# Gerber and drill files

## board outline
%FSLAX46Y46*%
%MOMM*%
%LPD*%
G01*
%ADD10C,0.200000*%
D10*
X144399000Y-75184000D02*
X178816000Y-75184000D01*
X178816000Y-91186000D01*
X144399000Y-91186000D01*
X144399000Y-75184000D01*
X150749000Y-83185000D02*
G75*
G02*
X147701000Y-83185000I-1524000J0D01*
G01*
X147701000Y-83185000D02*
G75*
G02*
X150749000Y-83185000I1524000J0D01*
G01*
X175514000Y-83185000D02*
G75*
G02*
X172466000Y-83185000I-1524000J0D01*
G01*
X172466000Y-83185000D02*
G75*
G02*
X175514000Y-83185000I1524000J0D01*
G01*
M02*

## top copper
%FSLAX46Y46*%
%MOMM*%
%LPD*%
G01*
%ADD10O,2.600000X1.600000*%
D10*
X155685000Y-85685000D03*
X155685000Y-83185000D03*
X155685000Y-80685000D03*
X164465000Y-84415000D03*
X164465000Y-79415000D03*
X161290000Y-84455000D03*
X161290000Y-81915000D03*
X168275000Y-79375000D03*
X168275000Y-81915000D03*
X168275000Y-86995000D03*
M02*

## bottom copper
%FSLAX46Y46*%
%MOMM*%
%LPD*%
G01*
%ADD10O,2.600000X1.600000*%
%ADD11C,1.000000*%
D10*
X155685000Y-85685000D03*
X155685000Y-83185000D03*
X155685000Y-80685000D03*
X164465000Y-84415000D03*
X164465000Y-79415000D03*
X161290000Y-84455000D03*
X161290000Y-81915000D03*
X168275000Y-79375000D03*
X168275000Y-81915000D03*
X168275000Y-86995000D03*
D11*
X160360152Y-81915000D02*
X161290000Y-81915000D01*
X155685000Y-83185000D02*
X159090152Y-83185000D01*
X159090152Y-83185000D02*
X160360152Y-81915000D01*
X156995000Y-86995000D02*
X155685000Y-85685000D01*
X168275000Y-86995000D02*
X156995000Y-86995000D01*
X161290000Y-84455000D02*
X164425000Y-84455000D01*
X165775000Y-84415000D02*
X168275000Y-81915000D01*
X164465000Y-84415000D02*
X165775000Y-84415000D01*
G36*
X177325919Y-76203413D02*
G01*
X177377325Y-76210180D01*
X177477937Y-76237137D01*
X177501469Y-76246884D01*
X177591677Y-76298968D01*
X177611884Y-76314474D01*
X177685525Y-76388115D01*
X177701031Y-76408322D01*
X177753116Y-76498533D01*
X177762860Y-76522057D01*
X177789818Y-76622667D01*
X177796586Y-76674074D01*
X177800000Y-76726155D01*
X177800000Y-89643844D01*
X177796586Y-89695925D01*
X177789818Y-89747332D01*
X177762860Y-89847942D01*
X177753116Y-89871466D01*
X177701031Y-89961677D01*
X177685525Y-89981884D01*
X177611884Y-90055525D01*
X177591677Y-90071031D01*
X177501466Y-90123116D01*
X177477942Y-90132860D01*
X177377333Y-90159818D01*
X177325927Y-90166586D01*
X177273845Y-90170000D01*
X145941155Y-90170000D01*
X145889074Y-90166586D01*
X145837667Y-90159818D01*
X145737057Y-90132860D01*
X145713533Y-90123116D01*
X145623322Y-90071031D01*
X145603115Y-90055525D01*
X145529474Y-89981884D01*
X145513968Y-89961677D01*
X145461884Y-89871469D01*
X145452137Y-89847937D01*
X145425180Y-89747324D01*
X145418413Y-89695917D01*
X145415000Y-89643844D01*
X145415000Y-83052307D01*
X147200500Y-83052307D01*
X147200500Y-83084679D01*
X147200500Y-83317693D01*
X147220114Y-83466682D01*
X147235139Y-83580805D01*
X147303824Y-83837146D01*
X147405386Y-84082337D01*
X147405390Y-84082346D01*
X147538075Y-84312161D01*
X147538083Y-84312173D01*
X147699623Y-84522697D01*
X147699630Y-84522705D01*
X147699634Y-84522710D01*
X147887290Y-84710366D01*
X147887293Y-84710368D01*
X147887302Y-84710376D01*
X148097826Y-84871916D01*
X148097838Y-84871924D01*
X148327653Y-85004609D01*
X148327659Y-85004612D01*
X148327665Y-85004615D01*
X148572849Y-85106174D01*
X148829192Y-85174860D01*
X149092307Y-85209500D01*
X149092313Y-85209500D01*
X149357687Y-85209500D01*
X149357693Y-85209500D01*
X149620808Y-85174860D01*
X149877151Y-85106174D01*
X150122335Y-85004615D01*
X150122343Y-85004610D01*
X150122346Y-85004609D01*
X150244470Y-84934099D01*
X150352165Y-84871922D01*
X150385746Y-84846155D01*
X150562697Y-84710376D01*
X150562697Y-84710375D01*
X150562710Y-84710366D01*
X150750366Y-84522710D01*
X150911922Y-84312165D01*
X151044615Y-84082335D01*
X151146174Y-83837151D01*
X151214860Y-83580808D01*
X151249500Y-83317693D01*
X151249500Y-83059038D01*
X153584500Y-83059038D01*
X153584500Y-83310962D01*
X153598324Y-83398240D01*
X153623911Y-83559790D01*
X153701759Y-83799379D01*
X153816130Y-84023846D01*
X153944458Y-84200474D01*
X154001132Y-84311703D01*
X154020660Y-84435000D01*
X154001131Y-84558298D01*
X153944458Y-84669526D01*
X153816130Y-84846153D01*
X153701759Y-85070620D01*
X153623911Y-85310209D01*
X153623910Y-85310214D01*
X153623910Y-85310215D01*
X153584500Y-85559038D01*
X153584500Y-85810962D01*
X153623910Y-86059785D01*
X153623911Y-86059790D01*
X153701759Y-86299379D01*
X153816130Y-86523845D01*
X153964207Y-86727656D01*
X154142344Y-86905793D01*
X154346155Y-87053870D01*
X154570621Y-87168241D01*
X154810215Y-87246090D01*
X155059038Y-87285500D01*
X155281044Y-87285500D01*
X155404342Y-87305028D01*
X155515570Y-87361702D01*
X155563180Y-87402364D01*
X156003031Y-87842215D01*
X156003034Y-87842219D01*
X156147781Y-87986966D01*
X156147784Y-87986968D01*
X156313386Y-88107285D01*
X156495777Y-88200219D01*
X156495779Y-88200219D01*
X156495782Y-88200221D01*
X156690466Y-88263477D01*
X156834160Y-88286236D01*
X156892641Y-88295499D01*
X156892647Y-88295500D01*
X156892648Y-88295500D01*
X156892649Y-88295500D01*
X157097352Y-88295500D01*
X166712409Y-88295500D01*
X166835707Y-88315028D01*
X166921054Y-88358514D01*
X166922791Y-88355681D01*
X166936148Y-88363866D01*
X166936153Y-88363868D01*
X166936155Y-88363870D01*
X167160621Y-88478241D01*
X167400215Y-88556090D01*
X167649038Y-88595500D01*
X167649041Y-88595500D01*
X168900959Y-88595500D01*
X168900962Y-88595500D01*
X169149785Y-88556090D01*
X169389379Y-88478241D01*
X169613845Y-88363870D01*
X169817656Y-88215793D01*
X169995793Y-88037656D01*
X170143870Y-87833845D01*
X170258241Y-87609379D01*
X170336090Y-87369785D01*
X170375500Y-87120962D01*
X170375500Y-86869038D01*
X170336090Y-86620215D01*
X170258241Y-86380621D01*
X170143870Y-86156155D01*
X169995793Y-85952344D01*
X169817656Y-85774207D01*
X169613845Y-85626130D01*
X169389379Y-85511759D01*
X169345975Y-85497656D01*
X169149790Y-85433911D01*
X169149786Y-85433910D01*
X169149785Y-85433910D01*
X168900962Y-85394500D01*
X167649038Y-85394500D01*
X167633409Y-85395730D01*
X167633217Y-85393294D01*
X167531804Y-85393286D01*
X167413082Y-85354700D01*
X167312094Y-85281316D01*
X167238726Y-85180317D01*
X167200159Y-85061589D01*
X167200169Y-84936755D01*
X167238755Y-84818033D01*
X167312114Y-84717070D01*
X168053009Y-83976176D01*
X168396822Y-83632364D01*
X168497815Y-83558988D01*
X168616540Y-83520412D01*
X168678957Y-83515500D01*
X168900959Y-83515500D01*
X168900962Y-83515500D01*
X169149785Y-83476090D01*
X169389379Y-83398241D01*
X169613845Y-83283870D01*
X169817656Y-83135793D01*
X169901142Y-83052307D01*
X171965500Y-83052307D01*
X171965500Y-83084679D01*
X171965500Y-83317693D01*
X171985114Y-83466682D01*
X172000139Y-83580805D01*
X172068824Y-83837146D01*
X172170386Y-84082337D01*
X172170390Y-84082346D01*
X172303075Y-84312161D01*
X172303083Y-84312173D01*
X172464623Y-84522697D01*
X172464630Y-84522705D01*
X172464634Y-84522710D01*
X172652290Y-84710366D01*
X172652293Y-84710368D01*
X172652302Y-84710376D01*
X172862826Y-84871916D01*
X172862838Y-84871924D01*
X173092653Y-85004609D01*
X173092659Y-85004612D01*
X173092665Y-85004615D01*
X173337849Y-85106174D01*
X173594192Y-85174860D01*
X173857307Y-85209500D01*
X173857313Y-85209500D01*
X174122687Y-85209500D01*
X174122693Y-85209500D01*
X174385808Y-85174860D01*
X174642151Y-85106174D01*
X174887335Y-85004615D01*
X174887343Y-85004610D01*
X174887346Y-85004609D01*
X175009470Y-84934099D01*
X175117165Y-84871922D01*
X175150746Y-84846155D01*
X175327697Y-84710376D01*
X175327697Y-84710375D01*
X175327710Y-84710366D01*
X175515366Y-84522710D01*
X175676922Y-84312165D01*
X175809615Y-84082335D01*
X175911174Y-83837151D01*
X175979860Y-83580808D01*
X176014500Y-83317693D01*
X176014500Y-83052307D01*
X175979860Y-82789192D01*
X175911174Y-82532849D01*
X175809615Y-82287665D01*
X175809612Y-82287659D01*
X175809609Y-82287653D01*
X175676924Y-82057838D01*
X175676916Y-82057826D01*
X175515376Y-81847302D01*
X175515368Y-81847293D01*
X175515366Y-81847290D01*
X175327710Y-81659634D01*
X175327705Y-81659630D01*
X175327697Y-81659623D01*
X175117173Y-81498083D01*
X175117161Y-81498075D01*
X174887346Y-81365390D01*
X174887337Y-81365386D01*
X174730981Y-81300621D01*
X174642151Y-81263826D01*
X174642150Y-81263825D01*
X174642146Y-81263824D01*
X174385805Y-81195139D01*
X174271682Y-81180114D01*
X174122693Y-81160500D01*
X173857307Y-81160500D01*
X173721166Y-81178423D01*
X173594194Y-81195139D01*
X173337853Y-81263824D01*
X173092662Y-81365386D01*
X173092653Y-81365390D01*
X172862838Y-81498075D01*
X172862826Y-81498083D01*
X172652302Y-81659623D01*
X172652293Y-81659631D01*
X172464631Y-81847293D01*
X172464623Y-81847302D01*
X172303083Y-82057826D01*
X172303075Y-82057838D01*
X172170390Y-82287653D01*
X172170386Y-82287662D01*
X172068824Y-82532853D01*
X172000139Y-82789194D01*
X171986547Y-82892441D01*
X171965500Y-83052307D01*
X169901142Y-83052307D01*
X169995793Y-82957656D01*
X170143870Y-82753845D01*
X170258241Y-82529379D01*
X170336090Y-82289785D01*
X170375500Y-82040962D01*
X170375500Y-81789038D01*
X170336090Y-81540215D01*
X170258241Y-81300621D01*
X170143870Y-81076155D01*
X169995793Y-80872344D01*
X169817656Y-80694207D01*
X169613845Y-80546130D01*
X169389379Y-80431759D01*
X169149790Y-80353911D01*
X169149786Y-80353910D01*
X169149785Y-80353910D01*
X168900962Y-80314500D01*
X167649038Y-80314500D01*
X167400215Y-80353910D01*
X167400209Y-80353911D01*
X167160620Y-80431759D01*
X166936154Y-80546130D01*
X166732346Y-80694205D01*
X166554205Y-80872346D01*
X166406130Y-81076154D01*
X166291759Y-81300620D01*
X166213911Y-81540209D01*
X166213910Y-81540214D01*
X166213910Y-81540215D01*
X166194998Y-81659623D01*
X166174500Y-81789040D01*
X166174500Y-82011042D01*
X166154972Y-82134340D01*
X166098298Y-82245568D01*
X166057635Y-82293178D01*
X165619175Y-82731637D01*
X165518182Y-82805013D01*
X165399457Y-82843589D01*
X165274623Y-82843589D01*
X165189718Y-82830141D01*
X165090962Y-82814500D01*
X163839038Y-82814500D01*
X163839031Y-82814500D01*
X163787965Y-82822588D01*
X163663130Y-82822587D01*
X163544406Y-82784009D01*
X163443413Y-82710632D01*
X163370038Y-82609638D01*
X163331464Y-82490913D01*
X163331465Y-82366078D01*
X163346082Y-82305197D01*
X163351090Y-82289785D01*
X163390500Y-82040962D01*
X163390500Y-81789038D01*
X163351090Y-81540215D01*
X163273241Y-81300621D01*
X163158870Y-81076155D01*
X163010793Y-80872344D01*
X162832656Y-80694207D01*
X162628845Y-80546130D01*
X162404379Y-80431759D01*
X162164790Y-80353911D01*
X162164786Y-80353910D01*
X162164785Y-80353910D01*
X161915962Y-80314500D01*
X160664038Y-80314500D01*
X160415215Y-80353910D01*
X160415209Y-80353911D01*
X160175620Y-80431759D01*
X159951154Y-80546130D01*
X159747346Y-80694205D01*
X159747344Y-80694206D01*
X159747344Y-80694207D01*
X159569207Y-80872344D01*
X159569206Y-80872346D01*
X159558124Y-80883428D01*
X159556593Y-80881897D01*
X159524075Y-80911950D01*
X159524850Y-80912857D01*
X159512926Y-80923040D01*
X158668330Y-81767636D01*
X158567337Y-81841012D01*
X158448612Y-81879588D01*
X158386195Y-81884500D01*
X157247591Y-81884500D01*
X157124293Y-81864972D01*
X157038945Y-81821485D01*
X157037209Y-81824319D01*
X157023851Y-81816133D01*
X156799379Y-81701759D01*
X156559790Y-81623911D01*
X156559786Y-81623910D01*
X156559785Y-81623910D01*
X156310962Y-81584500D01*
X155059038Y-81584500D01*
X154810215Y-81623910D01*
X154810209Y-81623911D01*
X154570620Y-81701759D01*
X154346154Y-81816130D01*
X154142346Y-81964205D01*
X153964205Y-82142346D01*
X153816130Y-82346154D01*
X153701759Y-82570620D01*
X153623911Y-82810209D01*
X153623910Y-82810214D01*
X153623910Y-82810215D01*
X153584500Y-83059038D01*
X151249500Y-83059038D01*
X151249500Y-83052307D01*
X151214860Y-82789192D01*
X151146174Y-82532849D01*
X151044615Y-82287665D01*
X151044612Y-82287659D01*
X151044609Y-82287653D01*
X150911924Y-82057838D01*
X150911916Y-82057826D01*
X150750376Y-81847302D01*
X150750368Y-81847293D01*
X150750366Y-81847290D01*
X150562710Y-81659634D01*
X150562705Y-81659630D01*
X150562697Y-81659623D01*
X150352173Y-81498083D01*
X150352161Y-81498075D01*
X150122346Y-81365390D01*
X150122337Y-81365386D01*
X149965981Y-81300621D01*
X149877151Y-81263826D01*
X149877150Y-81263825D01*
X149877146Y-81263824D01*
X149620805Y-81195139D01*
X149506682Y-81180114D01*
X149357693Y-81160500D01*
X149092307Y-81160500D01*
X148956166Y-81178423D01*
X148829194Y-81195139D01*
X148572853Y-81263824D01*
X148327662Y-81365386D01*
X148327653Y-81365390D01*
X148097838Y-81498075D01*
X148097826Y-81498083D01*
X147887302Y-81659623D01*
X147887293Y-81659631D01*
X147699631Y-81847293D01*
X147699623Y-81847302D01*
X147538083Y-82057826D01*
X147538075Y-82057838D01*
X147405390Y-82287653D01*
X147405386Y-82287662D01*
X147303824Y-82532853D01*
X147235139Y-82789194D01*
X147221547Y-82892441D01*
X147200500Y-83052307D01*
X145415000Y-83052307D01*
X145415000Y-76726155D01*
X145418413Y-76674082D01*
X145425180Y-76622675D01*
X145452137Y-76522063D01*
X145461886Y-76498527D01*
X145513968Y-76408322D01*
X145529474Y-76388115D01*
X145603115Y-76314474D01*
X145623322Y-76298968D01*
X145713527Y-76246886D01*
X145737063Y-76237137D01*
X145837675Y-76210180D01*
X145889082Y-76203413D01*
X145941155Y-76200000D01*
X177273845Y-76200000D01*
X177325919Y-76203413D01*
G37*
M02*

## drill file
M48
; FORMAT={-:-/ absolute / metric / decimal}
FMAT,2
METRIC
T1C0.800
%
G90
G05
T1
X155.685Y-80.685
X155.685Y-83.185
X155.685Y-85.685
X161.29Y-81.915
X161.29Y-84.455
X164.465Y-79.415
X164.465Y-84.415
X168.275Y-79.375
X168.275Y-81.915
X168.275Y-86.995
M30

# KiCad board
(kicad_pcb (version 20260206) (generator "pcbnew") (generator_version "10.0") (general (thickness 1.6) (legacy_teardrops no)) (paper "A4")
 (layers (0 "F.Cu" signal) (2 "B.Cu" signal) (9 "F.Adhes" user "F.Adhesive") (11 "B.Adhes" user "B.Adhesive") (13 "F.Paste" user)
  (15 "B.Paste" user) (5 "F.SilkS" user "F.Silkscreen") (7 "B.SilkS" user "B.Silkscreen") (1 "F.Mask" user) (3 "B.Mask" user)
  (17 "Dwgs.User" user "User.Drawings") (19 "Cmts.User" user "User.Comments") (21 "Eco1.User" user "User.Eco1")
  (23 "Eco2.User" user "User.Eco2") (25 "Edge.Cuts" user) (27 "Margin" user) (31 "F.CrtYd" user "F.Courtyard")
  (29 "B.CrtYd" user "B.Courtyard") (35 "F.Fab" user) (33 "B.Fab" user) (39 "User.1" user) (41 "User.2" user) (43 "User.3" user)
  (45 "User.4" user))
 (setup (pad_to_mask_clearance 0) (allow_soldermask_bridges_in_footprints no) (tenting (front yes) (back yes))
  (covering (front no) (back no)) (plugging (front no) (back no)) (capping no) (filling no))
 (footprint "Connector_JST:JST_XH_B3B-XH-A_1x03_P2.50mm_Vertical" (layer "F.Cu") (at 155.685 85.685 90)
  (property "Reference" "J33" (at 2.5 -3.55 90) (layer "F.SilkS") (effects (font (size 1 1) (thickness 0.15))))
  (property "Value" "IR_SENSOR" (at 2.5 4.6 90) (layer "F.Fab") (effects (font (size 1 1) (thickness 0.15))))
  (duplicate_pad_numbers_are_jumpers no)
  (pad "1" thru_hole oval (at 0 0 180) (size 2.6 1.6) (drill 0.8) (layers "*.Cu" "*.Mask") (remove_unused_layers no) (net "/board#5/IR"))
  (pad "2" thru_hole oval (at 2.5 0 180) (size 2.6 1.6) (drill 0.8) (layers "*.Cu" "*.Mask") (remove_unused_layers no)
   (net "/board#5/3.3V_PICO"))
  (pad "3" thru_hole oval (at 5 0 180) (size 2.6 1.6) (drill 0.8) (layers "*.Cu" "*.Mask") (remove_unused_layers no) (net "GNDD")))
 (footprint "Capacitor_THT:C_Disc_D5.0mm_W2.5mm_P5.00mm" (layer "F.Cu") (at 164.465 84.415 90)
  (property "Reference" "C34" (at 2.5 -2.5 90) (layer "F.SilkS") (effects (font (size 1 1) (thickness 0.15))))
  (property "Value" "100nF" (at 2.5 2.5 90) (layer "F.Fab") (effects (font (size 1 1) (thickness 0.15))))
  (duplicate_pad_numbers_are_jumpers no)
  (pad "1" thru_hole oval (at 0 0 180) (size 2.6 1.6) (drill 0.8) (layers "*.Cu" "*.Mask") (remove_unused_layers no) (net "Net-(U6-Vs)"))
  (pad "2" thru_hole oval (at 5 0 180) (size 2.6 1.6) (drill 0.8) (layers "*.Cu" "*.Mask") (remove_unused_layers no) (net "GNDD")))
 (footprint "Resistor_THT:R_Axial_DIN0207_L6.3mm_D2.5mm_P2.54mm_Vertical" (layer "F.Cu") (at 161.29 84.455 90)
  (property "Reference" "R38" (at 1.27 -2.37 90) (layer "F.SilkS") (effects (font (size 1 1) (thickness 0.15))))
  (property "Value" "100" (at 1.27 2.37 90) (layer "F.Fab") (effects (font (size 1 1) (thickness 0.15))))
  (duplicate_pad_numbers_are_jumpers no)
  (pad "1" thru_hole oval (at 0 0 180) (size 2.6 1.6) (drill 0.8) (layers "*.Cu" "*.Mask") (remove_unused_layers no) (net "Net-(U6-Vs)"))
  (pad "2" thru_hole oval (at 2.54 0 180) (size 2.6 1.6) (drill 0.8) (layers "*.Cu" "*.Mask") (remove_unused_layers no)
   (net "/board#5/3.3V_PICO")))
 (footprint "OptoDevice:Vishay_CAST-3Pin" (layer "B.Cu") (at 168.275 79.375 -90)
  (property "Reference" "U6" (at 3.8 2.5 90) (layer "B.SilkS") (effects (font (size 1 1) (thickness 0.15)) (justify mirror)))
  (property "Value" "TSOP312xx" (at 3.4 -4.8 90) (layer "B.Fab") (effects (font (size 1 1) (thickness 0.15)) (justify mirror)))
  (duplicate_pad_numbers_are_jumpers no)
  (pad "1" thru_hole oval (at 0 0 180) (size 2.6 1.6) (drill 0.8) (layers "*.Cu" "*.Mask") (remove_unused_layers no) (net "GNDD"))
  (pad "2" thru_hole oval (at 2.54 0 180) (size 2.6 1.6) (drill 0.8) (layers "*.Cu" "*.Mask") (remove_unused_layers no) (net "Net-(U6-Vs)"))
  (pad "3" thru_hole oval (at 7.62 0 180) (size 2.6 1.6) (drill 0.8) (layers "*.Cu" "*.Mask") (remove_unused_layers no) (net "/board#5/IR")))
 (gr_rect (start 144.399 75.184) (end 178.816 91.186) (stroke (width 0.2) (type solid)) (fill no) (layer "Edge.Cuts"))
 (gr_circle (center 149.225 83.185) (end 149.225 81.661) (stroke (width 0.2) (type solid)) (fill no) (layer "Edge.Cuts"))
 (gr_circle (center 173.99 83.185) (end 173.99 81.661) (stroke (width 0.2) (type solid)) (fill no) (layer "Edge.Cuts"))
 (segment (start 160.360152 81.915) (end 161.29 81.915) (width 1) (layer "B.Cu") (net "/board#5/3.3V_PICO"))
 (segment (start 155.685 83.185) (end 159.090152 83.185) (width 1) (layer "B.Cu") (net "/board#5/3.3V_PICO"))
 (segment (start 159.090152 83.185) (end 160.360152 81.915) (width 1) (layer "B.Cu") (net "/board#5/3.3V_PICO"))
 (segment (start 156.995 86.995) (end 155.685 85.685) (width 1) (layer "B.Cu") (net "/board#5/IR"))
 (segment (start 168.275 86.995) (end 156.995 86.995) (width 1) (layer "B.Cu") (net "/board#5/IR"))
 (segment (start 161.29 84.455) (end 164.425 84.455) (width 1) (layer "B.Cu") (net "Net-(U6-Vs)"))
 (segment (start 165.775 84.415) (end 168.275 81.915) (width 1) (layer "B.Cu") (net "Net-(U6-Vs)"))
 (segment (start 164.465 84.415) (end 165.775 84.415) (width 1) (layer "B.Cu") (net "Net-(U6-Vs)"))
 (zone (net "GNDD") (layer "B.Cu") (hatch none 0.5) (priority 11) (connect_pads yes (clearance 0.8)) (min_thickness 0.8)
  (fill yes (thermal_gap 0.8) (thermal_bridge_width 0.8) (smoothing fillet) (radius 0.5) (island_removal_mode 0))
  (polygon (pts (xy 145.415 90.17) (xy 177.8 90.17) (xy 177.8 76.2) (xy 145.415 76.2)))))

